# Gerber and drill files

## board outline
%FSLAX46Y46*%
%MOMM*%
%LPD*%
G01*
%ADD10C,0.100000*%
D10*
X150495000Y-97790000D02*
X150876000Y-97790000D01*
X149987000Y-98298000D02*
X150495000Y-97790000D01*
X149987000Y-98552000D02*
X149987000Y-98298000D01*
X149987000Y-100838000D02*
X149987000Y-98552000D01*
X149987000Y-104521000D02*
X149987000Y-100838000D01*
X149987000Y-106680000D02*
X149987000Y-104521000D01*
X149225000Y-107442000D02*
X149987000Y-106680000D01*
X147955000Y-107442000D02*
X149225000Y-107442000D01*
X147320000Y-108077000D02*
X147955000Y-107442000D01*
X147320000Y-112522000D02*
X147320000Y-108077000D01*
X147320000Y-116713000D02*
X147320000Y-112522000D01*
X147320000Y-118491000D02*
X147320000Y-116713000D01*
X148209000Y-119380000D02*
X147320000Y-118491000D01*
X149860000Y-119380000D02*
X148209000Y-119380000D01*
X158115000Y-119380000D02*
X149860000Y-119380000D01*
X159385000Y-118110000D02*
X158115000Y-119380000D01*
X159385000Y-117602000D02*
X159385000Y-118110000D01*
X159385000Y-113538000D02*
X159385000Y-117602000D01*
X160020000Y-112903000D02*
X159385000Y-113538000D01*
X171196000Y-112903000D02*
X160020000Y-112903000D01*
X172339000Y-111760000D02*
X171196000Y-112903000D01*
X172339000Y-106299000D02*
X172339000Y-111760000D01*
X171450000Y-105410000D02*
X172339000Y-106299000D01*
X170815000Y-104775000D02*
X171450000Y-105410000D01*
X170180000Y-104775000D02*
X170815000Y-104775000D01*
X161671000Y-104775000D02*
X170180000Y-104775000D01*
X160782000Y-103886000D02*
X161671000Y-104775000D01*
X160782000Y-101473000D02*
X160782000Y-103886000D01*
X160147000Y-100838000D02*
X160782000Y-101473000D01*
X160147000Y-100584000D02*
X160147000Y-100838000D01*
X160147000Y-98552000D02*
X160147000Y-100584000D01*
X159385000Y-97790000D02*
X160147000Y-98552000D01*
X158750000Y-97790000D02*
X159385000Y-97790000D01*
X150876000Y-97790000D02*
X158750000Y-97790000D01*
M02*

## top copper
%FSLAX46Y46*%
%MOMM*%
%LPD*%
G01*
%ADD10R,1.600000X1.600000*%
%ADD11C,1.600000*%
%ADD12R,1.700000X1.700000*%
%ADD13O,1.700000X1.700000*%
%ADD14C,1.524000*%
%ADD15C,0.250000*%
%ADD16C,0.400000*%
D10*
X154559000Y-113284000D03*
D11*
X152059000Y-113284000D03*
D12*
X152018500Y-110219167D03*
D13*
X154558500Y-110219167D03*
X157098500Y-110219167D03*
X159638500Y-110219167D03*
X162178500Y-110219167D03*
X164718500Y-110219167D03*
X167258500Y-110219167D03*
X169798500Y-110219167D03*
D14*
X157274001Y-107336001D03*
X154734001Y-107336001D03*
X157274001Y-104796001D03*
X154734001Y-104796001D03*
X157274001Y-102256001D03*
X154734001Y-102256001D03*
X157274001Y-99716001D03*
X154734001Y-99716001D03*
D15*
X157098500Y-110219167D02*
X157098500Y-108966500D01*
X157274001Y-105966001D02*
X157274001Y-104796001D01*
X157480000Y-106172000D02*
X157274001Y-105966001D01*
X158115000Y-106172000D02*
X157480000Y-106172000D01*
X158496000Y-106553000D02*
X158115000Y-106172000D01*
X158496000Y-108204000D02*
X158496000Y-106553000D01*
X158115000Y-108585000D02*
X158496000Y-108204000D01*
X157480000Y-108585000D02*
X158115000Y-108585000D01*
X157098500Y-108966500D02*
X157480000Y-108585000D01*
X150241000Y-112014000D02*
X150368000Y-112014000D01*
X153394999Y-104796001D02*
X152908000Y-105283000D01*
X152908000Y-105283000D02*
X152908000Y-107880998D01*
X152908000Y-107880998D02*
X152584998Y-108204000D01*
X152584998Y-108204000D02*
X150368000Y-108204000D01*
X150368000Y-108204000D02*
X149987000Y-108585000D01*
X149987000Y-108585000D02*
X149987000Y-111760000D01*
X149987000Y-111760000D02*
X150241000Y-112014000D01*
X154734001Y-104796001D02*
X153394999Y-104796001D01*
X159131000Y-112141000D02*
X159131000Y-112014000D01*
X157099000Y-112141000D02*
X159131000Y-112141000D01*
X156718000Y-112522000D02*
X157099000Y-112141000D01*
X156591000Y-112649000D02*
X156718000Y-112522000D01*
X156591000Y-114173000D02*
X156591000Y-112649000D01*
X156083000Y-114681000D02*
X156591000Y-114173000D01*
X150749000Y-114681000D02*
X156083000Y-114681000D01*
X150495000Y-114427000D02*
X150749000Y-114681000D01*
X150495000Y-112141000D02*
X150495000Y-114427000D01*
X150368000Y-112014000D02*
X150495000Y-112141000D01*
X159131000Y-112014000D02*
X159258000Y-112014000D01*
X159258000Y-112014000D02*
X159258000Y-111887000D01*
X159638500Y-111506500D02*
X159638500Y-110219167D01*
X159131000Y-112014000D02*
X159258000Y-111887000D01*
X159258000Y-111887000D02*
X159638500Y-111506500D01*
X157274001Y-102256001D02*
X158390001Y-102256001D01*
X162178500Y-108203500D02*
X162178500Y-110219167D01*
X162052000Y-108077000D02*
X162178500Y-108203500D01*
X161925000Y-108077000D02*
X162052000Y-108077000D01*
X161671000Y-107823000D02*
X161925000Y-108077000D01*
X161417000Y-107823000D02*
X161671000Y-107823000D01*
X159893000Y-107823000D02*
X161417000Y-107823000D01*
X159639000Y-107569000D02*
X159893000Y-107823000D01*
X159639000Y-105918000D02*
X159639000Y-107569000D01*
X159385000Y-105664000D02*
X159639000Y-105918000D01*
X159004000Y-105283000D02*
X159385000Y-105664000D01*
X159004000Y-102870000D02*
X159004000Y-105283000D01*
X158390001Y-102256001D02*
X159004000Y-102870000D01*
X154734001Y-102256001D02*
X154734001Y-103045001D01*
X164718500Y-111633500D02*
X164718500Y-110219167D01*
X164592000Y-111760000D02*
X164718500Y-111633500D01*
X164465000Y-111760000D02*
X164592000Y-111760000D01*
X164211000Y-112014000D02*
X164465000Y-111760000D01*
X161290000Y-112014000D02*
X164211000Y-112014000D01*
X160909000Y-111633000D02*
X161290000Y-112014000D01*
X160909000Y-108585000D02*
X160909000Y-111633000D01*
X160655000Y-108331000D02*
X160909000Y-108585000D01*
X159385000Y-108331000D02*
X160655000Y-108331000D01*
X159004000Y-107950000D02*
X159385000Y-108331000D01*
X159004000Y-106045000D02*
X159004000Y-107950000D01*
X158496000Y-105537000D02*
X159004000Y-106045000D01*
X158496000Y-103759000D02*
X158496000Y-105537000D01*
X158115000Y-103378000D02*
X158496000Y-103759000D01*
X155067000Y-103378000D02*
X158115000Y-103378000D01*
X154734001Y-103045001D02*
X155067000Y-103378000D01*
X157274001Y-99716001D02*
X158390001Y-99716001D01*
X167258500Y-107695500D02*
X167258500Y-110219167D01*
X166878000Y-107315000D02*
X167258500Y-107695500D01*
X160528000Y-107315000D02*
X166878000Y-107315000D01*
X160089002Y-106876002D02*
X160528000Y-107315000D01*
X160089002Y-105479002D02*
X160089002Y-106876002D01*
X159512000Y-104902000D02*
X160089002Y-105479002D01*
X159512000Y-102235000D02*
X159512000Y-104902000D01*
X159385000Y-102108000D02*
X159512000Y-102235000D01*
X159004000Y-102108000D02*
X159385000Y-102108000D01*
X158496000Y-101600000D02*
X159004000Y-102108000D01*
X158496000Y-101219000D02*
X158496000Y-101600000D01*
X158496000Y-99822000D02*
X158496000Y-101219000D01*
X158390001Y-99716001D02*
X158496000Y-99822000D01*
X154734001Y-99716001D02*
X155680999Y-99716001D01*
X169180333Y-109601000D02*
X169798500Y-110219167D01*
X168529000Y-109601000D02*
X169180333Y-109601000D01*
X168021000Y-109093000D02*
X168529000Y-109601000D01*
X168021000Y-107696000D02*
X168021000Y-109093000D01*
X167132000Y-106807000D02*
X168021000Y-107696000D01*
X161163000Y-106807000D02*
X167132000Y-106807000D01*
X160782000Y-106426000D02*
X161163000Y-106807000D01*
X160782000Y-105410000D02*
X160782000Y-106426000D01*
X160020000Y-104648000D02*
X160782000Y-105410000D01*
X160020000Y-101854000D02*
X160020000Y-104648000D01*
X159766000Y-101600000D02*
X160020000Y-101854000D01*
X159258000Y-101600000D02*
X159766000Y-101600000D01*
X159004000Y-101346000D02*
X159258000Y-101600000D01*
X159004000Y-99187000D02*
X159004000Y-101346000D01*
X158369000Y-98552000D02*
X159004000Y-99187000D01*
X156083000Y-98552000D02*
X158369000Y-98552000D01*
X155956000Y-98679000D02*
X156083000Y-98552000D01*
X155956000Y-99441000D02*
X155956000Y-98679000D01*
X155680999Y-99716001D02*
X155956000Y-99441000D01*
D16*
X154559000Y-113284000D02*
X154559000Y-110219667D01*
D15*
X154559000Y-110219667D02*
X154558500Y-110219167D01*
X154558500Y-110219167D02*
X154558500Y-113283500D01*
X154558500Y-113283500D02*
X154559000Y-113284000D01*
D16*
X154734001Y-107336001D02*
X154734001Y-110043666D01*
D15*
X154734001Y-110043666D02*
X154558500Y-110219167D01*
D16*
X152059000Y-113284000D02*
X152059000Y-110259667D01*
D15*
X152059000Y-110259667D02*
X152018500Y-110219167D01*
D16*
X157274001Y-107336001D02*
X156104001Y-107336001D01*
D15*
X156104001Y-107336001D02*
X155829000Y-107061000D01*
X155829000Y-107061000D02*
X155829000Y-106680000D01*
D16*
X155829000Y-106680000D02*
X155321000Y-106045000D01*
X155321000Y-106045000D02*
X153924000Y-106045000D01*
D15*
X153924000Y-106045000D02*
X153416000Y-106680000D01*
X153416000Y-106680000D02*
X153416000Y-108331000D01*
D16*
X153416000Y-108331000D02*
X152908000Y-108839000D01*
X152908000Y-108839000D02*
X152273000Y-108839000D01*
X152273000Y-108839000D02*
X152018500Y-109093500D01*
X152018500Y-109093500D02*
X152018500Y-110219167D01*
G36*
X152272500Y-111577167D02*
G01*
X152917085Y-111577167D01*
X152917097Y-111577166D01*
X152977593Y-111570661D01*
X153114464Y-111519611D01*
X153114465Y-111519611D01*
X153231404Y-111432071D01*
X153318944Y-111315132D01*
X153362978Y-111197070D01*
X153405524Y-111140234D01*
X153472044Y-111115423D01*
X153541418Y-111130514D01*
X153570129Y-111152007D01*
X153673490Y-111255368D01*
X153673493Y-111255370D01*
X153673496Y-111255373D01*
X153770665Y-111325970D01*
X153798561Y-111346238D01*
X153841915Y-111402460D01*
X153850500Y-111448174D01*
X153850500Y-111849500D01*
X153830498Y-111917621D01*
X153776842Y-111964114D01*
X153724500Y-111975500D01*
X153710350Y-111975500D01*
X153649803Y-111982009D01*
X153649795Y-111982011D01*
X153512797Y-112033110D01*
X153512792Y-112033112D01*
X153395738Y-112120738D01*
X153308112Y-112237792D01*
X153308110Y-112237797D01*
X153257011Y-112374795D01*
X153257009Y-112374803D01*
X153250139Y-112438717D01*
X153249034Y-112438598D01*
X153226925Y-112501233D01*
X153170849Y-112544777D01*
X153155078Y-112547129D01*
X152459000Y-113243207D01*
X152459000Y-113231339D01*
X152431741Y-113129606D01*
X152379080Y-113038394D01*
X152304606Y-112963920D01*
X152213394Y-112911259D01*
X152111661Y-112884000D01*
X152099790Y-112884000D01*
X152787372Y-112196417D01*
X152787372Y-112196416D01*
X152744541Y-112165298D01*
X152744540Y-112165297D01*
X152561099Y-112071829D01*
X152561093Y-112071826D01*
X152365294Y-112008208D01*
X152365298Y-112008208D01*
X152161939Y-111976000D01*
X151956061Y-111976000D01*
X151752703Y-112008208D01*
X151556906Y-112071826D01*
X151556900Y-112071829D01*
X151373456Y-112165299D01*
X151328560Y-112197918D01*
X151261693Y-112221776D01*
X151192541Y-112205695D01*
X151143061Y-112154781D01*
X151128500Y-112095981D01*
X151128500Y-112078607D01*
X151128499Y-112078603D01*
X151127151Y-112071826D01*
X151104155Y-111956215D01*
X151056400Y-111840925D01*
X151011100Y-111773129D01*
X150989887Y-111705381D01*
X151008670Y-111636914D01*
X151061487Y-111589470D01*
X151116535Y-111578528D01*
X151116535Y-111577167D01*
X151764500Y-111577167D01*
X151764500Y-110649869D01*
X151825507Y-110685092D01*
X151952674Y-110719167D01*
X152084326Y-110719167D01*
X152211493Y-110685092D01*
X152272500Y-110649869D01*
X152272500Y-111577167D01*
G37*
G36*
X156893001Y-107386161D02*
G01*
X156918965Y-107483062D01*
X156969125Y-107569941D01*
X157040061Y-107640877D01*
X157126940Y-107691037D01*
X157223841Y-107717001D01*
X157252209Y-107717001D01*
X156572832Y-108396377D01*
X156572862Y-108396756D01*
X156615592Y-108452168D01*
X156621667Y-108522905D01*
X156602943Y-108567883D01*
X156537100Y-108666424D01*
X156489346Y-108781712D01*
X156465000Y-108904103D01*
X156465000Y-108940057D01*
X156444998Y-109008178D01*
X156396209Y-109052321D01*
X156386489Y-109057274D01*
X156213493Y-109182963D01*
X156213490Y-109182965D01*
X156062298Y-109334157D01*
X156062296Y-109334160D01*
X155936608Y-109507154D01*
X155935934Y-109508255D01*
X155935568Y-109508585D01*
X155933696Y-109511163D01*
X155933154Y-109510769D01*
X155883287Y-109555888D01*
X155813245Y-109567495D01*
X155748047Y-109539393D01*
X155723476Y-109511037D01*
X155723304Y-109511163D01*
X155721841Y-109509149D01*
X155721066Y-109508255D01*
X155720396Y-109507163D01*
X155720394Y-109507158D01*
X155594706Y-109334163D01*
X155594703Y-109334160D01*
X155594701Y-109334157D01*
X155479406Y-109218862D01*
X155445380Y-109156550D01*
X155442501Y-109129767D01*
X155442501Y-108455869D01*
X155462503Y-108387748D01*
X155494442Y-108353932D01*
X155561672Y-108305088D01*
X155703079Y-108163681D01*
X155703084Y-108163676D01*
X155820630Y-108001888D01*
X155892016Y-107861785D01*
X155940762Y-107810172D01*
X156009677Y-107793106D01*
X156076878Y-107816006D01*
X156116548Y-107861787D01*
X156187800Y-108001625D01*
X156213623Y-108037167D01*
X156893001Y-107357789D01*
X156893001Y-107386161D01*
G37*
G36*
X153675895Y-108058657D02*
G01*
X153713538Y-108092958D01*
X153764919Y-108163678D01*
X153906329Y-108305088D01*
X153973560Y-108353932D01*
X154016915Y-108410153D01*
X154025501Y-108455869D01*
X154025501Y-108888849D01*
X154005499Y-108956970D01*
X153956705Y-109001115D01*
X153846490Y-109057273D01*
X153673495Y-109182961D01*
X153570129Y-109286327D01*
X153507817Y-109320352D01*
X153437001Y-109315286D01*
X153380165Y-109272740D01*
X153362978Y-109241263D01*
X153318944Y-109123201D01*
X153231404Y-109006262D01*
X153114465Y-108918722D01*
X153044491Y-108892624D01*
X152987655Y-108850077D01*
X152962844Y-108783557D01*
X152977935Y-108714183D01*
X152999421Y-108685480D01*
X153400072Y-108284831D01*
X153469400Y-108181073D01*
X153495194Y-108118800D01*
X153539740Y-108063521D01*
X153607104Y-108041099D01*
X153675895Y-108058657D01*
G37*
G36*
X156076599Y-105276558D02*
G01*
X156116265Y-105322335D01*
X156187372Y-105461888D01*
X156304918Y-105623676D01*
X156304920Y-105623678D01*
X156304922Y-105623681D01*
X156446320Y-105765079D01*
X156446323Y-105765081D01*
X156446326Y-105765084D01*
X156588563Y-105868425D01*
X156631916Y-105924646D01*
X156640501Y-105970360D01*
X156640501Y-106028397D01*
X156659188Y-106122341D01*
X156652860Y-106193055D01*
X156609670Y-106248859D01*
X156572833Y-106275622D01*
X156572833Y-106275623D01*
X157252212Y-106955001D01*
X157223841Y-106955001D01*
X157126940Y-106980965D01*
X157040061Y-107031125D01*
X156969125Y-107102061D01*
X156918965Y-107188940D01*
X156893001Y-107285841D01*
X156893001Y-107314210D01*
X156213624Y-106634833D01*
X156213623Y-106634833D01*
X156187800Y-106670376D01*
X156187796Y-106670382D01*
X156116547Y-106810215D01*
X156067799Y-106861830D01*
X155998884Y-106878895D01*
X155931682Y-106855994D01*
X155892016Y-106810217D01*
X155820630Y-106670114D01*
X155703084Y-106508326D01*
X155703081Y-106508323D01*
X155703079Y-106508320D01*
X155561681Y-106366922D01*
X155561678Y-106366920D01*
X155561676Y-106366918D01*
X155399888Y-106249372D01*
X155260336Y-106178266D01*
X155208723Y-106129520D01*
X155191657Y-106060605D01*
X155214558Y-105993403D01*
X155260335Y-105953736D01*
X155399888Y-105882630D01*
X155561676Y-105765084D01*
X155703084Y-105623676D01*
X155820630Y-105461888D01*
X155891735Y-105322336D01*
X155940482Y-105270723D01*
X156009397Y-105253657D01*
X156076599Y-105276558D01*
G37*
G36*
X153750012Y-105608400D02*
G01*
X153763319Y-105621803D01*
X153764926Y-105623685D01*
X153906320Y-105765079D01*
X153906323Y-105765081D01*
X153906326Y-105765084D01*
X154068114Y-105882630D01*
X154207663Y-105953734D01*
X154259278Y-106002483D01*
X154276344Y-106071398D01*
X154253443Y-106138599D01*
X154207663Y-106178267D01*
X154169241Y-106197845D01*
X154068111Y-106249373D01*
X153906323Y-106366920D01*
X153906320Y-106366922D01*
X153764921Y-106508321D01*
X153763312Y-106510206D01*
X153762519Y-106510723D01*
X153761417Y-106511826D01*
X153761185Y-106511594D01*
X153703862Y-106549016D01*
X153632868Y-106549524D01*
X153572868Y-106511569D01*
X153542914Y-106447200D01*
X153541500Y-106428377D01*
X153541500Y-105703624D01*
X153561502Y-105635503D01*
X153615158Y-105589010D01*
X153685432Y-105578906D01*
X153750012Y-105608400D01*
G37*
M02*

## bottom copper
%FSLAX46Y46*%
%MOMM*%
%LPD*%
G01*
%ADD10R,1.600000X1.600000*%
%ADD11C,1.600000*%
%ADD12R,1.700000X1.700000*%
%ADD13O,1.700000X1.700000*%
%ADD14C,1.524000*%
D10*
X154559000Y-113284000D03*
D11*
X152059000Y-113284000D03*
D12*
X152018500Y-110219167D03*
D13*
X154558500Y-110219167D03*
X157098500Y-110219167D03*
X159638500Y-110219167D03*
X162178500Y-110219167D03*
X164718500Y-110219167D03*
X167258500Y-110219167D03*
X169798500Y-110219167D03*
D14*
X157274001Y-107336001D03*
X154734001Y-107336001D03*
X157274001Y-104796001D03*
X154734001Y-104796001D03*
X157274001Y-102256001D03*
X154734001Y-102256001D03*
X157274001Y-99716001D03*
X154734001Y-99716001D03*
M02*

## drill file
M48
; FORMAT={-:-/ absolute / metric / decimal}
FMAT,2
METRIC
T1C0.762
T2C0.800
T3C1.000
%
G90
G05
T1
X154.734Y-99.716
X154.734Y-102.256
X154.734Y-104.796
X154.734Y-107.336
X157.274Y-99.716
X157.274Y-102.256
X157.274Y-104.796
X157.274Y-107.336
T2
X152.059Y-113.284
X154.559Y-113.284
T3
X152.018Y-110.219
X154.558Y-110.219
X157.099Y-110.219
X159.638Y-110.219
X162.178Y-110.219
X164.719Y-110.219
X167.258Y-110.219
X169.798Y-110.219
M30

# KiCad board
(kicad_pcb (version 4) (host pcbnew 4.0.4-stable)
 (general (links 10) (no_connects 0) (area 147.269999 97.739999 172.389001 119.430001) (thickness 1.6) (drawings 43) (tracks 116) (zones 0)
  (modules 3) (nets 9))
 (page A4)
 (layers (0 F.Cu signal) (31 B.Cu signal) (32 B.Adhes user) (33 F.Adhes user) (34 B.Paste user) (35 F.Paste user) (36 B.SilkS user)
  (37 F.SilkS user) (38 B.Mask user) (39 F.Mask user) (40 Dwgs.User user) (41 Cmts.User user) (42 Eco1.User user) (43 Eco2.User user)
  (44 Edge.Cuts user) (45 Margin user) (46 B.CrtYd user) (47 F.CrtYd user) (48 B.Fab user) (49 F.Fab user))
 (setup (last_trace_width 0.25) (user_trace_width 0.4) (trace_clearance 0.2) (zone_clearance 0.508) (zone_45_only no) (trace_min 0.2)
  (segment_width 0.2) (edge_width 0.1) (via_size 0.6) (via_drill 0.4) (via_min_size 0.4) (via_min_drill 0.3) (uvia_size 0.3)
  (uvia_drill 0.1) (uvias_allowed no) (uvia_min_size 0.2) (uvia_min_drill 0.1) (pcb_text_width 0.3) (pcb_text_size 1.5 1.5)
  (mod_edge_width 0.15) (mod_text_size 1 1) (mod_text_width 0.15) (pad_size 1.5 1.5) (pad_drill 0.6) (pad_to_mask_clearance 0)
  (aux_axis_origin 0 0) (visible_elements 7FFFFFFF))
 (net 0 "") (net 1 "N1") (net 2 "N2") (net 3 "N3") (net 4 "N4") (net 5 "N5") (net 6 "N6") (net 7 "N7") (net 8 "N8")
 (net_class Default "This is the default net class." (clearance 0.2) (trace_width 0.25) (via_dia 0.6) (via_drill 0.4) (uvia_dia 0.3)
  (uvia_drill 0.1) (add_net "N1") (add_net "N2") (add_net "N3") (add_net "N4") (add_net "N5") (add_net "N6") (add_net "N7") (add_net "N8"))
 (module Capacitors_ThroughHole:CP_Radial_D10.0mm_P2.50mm (layer F.Cu) (at 154.559 113.284 180)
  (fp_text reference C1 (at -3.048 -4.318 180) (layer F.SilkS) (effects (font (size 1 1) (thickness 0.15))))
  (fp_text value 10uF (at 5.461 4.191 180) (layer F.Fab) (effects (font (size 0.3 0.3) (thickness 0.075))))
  (pad 1 thru_hole rect (at 0 0 180) (size 1.6 1.6) (drill 0.8) (layers *.Cu *.Mask) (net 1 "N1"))
  (pad 2 thru_hole circle (at 2.5 0 180) (size 1.6 1.6) (drill 0.8) (layers *.Cu *.Mask) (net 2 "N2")))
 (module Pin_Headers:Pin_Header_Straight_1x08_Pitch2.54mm (layer F.Cu) (at 152.0185 110.219167 90)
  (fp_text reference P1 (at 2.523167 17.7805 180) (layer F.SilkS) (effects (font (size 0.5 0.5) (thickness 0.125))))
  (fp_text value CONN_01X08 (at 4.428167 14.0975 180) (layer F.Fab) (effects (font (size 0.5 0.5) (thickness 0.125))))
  (pad 1 thru_hole rect (at 0 0 90) (size 1.7 1.7) (drill 1) (layers *.Cu *.Mask) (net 2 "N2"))
  (pad 2 thru_hole oval (at 0 2.54 90) (size 1.7 1.7) (drill 1) (layers *.Cu *.Mask) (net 1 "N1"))
  (pad 3 thru_hole oval (at 0 5.08 90) (size 1.7 1.7) (drill 1) (layers *.Cu *.Mask) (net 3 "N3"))
  (pad 4 thru_hole oval (at 0 7.62 90) (size 1.7 1.7) (drill 1) (layers *.Cu *.Mask) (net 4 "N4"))
  (pad 5 thru_hole oval (at 0 10.16 90) (size 1.7 1.7) (drill 1) (layers *.Cu *.Mask) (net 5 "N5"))
  (pad 6 thru_hole oval (at 0 12.7 90) (size 1.7 1.7) (drill 1) (layers *.Cu *.Mask) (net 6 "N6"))
  (pad 7 thru_hole oval (at 0 15.24 90) (size 1.7 1.7) (drill 1) (layers *.Cu *.Mask) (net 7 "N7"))
  (pad 8 thru_hole oval (at 0 17.78 90) (size 1.7 1.7) (drill 1) (layers *.Cu *.Mask) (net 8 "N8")))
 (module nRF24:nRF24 (layer F.Cu) (at 154.734001 103.780001)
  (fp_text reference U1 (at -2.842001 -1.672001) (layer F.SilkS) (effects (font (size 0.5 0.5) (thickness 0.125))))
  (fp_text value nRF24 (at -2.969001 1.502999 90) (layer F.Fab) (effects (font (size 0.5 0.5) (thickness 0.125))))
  (pad 1 thru_hole circle (at 2.54 3.556) (size 1.524 1.524) (drill 0.762) (layers *.Cu *.Mask) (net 2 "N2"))
  (pad 2 thru_hole circle (at 0 3.556) (size 1.524 1.524) (drill 0.762) (layers *.Cu *.Mask) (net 1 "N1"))
  (pad 3 thru_hole circle (at 2.54 1.016) (size 1.524 1.524) (drill 0.762) (layers *.Cu *.Mask) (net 3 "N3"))
  (pad 4 thru_hole circle (at 0 1.016) (size 1.524 1.524) (drill 0.762) (layers *.Cu *.Mask) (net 4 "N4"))
  (pad 5 thru_hole circle (at 2.54 -1.524) (size 1.524 1.524) (drill 0.762) (layers *.Cu *.Mask) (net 5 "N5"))
  (pad 6 thru_hole circle (at 0 -1.524) (size 1.524 1.524) (drill 0.762) (layers *.Cu *.Mask) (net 6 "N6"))
  (pad 7 thru_hole circle (at 2.54 -4.064) (size 1.524 1.524) (drill 0.762) (layers *.Cu *.Mask) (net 7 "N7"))
  (pad 8 thru_hole circle (at 0 -4.064) (size 1.524 1.524) (drill 0.762) (layers *.Cu *.Mask) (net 8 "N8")))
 (gr_line (start 150.495 97.79) (end 150.876 97.79) (angle 90) (layer Edge.Cuts) (width 0.1))
 (gr_line (start 149.987 98.298) (end 150.495 97.79) (angle 90) (layer Edge.Cuts) (width 0.1))
 (gr_line (start 149.987 98.552) (end 149.987 98.298) (angle 90) (layer Edge.Cuts) (width 0.1))
 (gr_line (start 149.987 100.838) (end 149.987 98.552) (angle 90) (layer Edge.Cuts) (width 0.1))
 (gr_line (start 149.987 104.521) (end 149.987 100.838) (angle 90) (layer Edge.Cuts) (width 0.1))
 (gr_line (start 149.987 106.68) (end 149.987 104.521) (angle 90) (layer Edge.Cuts) (width 0.1))
 (gr_line (start 149.225 107.442) (end 149.987 106.68) (angle 90) (layer Edge.Cuts) (width 0.1))
 (gr_line (start 147.955 107.442) (end 149.225 107.442) (angle 90) (layer Edge.Cuts) (width 0.1))
 (gr_line (start 147.32 108.077) (end 147.955 107.442) (angle 90) (layer Edge.Cuts) (width 0.1))
 (gr_line (start 147.32 112.522) (end 147.32 108.077) (angle 90) (layer Edge.Cuts) (width 0.1))
 (gr_line (start 147.32 116.713) (end 147.32 112.522) (angle 90) (layer Edge.Cuts) (width 0.1))
 (gr_line (start 147.32 118.491) (end 147.32 116.713) (angle 90) (layer Edge.Cuts) (width 0.1))
 (gr_line (start 148.209 119.38) (end 147.32 118.491) (angle 90) (layer Edge.Cuts) (width 0.1))
 (gr_line (start 149.86 119.38) (end 148.209 119.38) (angle 90) (layer Edge.Cuts) (width 0.1))
 (gr_line (start 158.115 119.38) (end 149.86 119.38) (angle 90) (layer Edge.Cuts) (width 0.1))
 (gr_line (start 159.385 118.11) (end 158.115 119.38) (angle 90) (layer Edge.Cuts) (width 0.1))
 (gr_line (start 159.385 117.602) (end 159.385 118.11) (angle 90) (layer Edge.Cuts) (width 0.1))
 (gr_line (start 159.385 113.538) (end 159.385 117.602) (angle 90) (layer Edge.Cuts) (width 0.1))
 (gr_line (start 160.02 112.903) (end 159.385 113.538) (angle 90) (layer Edge.Cuts) (width 0.1))
 (gr_line (start 171.196 112.903) (end 160.02 112.903) (angle 90) (layer Edge.Cuts) (width 0.1))
 (gr_line (start 172.339 111.76) (end 171.196 112.903) (angle 90) (layer Edge.Cuts) (width 0.1))
 (gr_line (start 172.339 106.299) (end 172.339 111.76) (angle 90) (layer Edge.Cuts) (width 0.1))
 (gr_line (start 171.45 105.41) (end 172.339 106.299) (angle 90) (layer Edge.Cuts) (width 0.1))
 (gr_line (start 170.815 104.775) (end 171.45 105.41) (angle 90) (layer Edge.Cuts) (width 0.1))
 (gr_line (start 170.18 104.775) (end 170.815 104.775) (angle 90) (layer Edge.Cuts) (width 0.1))
 (gr_line (start 161.671 104.775) (end 170.18 104.775) (angle 90) (layer Edge.Cuts) (width 0.1))
 (gr_line (start 160.782 103.886) (end 161.671 104.775) (angle 90) (layer Edge.Cuts) (width 0.1))
 (gr_line (start 160.782 101.473) (end 160.782 103.886) (angle 90) (layer Edge.Cuts) (width 0.1))
 (gr_line (start 160.147 100.838) (end 160.782 101.473) (angle 90) (layer Edge.Cuts) (width 0.1))
 (gr_line (start 160.147 100.584) (end 160.147 100.838) (angle 90) (layer Edge.Cuts) (width 0.1))
 (gr_line (start 160.147 98.552) (end 160.147 100.584) (angle 90) (layer Edge.Cuts) (width 0.1))
 (gr_line (start 159.385 97.79) (end 160.147 98.552) (angle 90) (layer Edge.Cuts) (width 0.1))
 (gr_line (start 158.75 97.79) (end 159.385 97.79) (angle 90) (layer Edge.Cuts) (width 0.1))
 (gr_line (start 150.876 97.79) (end 158.75 97.79) (angle 90) (layer Edge.Cuts) (width 0.1))
 (segment (start 157.0985 110.219167) (end 157.0985 108.9665) (width 0.25) (layer F.Cu) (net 3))
 (segment (start 157.274001 105.966001) (end 157.274001 104.796001) (width 0.25) (layer F.Cu) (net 3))
 (segment (start 157.48 106.172) (end 157.274001 105.966001) (width 0.25) (layer F.Cu) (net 3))
 (segment (start 158.115 106.172) (end 157.48 106.172) (width 0.25) (layer F.Cu) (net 3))
 (segment (start 158.496 106.553) (end 158.115 106.172) (width 0.25) (layer F.Cu) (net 3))
 (segment (start 158.496 108.204) (end 158.496 106.553) (width 0.25) (layer F.Cu) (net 3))
 (segment (start 158.115 108.585) (end 158.496 108.204) (width 0.25) (layer F.Cu) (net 3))
 (segment (start 157.48 108.585) (end 158.115 108.585) (width 0.25) (layer F.Cu) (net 3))
 (segment (start 157.0985 108.9665) (end 157.48 108.585) (width 0.25) (layer F.Cu) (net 3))
 (segment (start 150.241 112.014) (end 150.368 112.014) (width 0.25) (layer F.Cu) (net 4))
 (segment (start 153.394999 104.796001) (end 152.908 105.283) (width 0.25) (layer F.Cu) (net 4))
 (segment (start 152.908 105.283) (end 152.908 107.880998) (width 0.25) (layer F.Cu) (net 4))
 (segment (start 152.908 107.880998) (end 152.584998 108.204) (width 0.25) (layer F.Cu) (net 4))
 (segment (start 152.584998 108.204) (end 150.368 108.204) (width 0.25) (layer F.Cu) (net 4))
 (segment (start 150.368 108.204) (end 149.987 108.585) (width 0.25) (layer F.Cu) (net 4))
 (segment (start 149.987 108.585) (end 149.987 111.76) (width 0.25) (layer F.Cu) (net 4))
 (segment (start 149.987 111.76) (end 150.241 112.014) (width 0.25) (layer F.Cu) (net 4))
 (segment (start 154.734001 104.796001) (end 153.394999 104.796001) (width 0.25) (layer F.Cu) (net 4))
 (segment (start 159.131 112.141) (end 159.131 112.014) (width 0.25) (layer F.Cu) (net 4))
 (segment (start 157.099 112.141) (end 159.131 112.141) (width 0.25) (layer F.Cu) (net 4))
 (segment (start 156.718 112.522) (end 157.099 112.141) (width 0.25) (layer F.Cu) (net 4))
 (segment (start 156.591 112.649) (end 156.718 112.522) (width 0.25) (layer F.Cu) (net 4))
 (segment (start 156.591 114.173) (end 156.591 112.649) (width 0.25) (layer F.Cu) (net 4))
 (segment (start 156.083 114.681) (end 156.591 114.173) (width 0.25) (layer F.Cu) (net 4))
 (segment (start 150.749 114.681) (end 156.083 114.681) (width 0.25) (layer F.Cu) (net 4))
 (segment (start 150.495 114.427) (end 150.749 114.681) (width 0.25) (layer F.Cu) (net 4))
 (segment (start 150.495 112.141) (end 150.495 114.427) (width 0.25) (layer F.Cu) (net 4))
 (segment (start 150.368 112.014) (end 150.495 112.141) (width 0.25) (layer F.Cu) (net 4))
 (segment (start 159.131 112.014) (end 159.258 112.014) (width 0.25) (layer F.Cu) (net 4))
 (segment (start 159.258 112.014) (end 159.258 111.887) (width 0.25) (layer F.Cu) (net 4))
 (segment (start 159.6385 111.5065) (end 159.6385 110.219167) (width 0.25) (layer F.Cu) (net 4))
 (segment (start 159.131 112.014) (end 159.258 111.887) (width 0.25) (layer F.Cu) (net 4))
 (segment (start 159.258 111.887) (end 159.6385 111.5065) (width 0.25) (layer F.Cu) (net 4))
 (segment (start 157.274001 102.256001) (end 158.390001 102.256001) (width 0.25) (layer F.Cu) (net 5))
 (segment (start 162.1785 108.2035) (end 162.1785 110.219167) (width 0.25) (layer F.Cu) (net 5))
 (segment (start 162.052 108.077) (end 162.1785 108.2035) (width 0.25) (layer F.Cu) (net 5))
 (segment (start 161.925 108.077) (end 162.052 108.077) (width 0.25) (layer F.Cu) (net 5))
 (segment (start 161.671 107.823) (end 161.925 108.077) (width 0.25) (layer F.Cu) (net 5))
 (segment (start 161.417 107.823) (end 161.671 107.823) (width 0.25) (layer F.Cu) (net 5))
 (segment (start 159.893 107.823) (end 161.417 107.823) (width 0.25) (layer F.Cu) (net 5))
 (segment (start 159.639 107.569) (end 159.893 107.823) (width 0.25) (layer F.Cu) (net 5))
 (segment (start 159.639 105.918) (end 159.639 107.569) (width 0.25) (layer F.Cu) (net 5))
 (segment (start 159.385 105.664) (end 159.639 105.918) (width 0.25) (layer F.Cu) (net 5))
 (segment (start 159.004 105.283) (end 159.385 105.664) (width 0.25) (layer F.Cu) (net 5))
 (segment (start 159.004 102.87) (end 159.004 105.283) (width 0.25) (layer F.Cu) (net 5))
 (segment (start 158.390001 102.256001) (end 159.004 102.87) (width 0.25) (layer F.Cu) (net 5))
 (segment (start 154.734001 102.256001) (end 154.734001 103.045001) (width 0.25) (layer F.Cu) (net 6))
 (segment (start 164.7185 111.6335) (end 164.7185 110.219167) (width 0.25) (layer F.Cu) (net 6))
 (segment (start 164.592 111.76) (end 164.7185 111.6335) (width 0.25) (layer F.Cu) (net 6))
 (segment (start 164.465 111.76) (end 164.592 111.76) (width 0.25) (layer F.Cu) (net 6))
 (segment (start 164.211 112.014) (end 164.465 111.76) (width 0.25) (layer F.Cu) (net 6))
 (segment (start 161.29 112.014) (end 164.211 112.014) (width 0.25) (layer F.Cu) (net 6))
 (segment (start 160.909 111.633) (end 161.29 112.014) (width 0.25) (layer F.Cu) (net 6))
 (segment (start 160.909 108.585) (end 160.909 111.633) (width 0.25) (layer F.Cu) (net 6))
 (segment (start 160.655 108.331) (end 160.909 108.585) (width 0.25) (layer F.Cu) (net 6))
 (segment (start 159.385 108.331) (end 160.655 108.331) (width 0.25) (layer F.Cu) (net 6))
 (segment (start 159.004 107.95) (end 159.385 108.331) (width 0.25) (layer F.Cu) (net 6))
 (segment (start 159.004 106.045) (end 159.004 107.95) (width 0.25) (layer F.Cu) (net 6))
 (segment (start 158.496 105.537) (end 159.004 106.045) (width 0.25) (layer F.Cu) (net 6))
 (segment (start 158.496 103.759) (end 158.496 105.537) (width 0.25) (layer F.Cu) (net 6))
 (segment (start 158.115 103.378) (end 158.496 103.759) (width 0.25) (layer F.Cu) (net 6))
 (segment (start 155.067 103.378) (end 158.115 103.378) (width 0.25) (layer F.Cu) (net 6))
 (segment (start 154.734001 103.045001) (end 155.067 103.378) (width 0.25) (layer F.Cu) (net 6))
 (segment (start 157.274001 99.716001) (end 158.390001 99.716001) (width 0.25) (layer F.Cu) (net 7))
 (segment (start 167.2585 107.6955) (end 167.2585 110.219167) (width 0.25) (layer F.Cu) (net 7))
 (segment (start 166.878 107.315) (end 167.2585 107.6955) (width 0.25) (layer F.Cu) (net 7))
 (segment (start 160.528 107.315) (end 166.878 107.315) (width 0.25) (layer F.Cu) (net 7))
 (segment (start 160.089002 106.876002) (end 160.528 107.315) (width 0.25) (layer F.Cu) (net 7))
 (segment (start 160.089002 105.479002) (end 160.089002 106.876002) (width 0.25) (layer F.Cu) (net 7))
 (segment (start 159.512 104.902) (end 160.089002 105.479002) (width 0.25) (layer F.Cu) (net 7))
 (segment (start 159.512 102.235) (end 159.512 104.902) (width 0.25) (layer F.Cu) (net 7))
 (segment (start 159.385 102.108) (end 159.512 102.235) (width 0.25) (layer F.Cu) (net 7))
 (segment (start 159.004 102.108) (end 159.385 102.108) (width 0.25) (layer F.Cu) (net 7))
 (segment (start 158.496 101.6) (end 159.004 102.108) (width 0.25) (layer F.Cu) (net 7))
 (segment (start 158.496 101.219) (end 158.496 101.6) (width 0.25) (layer F.Cu) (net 7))
 (segment (start 158.496 99.822) (end 158.496 101.219) (width 0.25) (layer F.Cu) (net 7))
 (segment (start 158.390001 99.716001) (end 158.496 99.822) (width 0.25) (layer F.Cu) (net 7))
 (segment (start 154.734001 99.716001) (end 155.680999 99.716001) (width 0.25) (layer F.Cu) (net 8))
 (segment (start 169.180333 109.601) (end 169.7985 110.219167) (width 0.25) (layer F.Cu) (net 8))
 (segment (start 168.529 109.601) (end 169.180333 109.601) (width 0.25) (layer F.Cu) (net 8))
 (segment (start 168.021 109.093) (end 168.529 109.601) (width 0.25) (layer F.Cu) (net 8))
 (segment (start 168.021 107.696) (end 168.021 109.093) (width 0.25) (layer F.Cu) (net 8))
 (segment (start 167.132 106.807) (end 168.021 107.696) (width 0.25) (layer F.Cu) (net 8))
 (segment (start 161.163 106.807) (end 167.132 106.807) (width 0.25) (layer F.Cu) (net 8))
 (segment (start 160.782 106.426) (end 161.163 106.807) (width 0.25) (layer F.Cu) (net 8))
 (segment (start 160.782 105.41) (end 160.782 106.426) (width 0.25) (layer F.Cu) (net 8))
 (segment (start 160.02 104.648) (end 160.782 105.41) (width 0.25) (layer F.Cu) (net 8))
 (segment (start 160.02 101.854) (end 160.02 104.648) (width 0.25) (layer F.Cu) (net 8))
 (segment (start 159.766 101.6) (end 160.02 101.854) (width 0.25) (layer F.Cu) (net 8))
 (segment (start 159.258 101.6) (end 159.766 101.6) (width 0.25) (layer F.Cu) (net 8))
 (segment (start 159.004 101.346) (end 159.258 101.6) (width 0.25) (layer F.Cu) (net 8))
 (segment (start 159.004 99.187) (end 159.004 101.346) (width 0.25) (layer F.Cu) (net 8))
 (segment (start 158.369 98.552) (end 159.004 99.187) (width 0.25) (layer F.Cu) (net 8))
 (segment (start 156.083 98.552) (end 158.369 98.552) (width 0.25) (layer F.Cu) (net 8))
 (segment (start 155.956 98.679) (end 156.083 98.552) (width 0.25) (layer F.Cu) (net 8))
 (segment (start 155.956 99.441) (end 155.956 98.679) (width 0.25) (layer F.Cu) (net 8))
 (segment (start 155.680999 99.716001) (end 155.956 99.441) (width 0.25) (layer F.Cu) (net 8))
 (segment (start 154.559 113.284) (end 154.559 110.219667) (width 0.4) (layer F.Cu) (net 1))
 (segment (start 154.559 110.219667) (end 154.5585 110.219167) (width 0.25) (layer F.Cu) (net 1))
 (segment (start 154.5585 110.219167) (end 154.5585 113.2835) (width 0.25) (layer F.Cu) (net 1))
 (segment (start 154.5585 113.2835) (end 154.559 113.284) (width 0.25) (layer F.Cu) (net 1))
 (segment (start 154.734001 107.336001) (end 154.734001 110.043666) (width 0.4) (layer F.Cu) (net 1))
 (segment (start 154.734001 110.043666) (end 154.5585 110.219167) (width 0.25) (layer F.Cu) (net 1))
 (segment (start 152.059 113.284) (end 152.059 110.259667) (width 0.4) (layer F.Cu) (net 2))
 (segment (start 152.059 110.259667) (end 152.0185 110.219167) (width 0.25) (layer F.Cu) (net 2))
 (segment (start 157.274001 107.336001) (end 156.104001 107.336001) (width 0.4) (layer F.Cu) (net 2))
 (segment (start 156.104001 107.336001) (end 155.829 107.061) (width 0.25) (layer F.Cu) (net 2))
 (segment (start 155.829 107.061) (end 155.829 106.68) (width 0.25) (layer F.Cu) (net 2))
 (segment (start 155.829 106.68) (end 155.321 106.045) (width 0.4) (layer F.Cu) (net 2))
 (segment (start 155.321 106.045) (end 153.924 106.045) (width 0.4) (layer F.Cu) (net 2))
 (segment (start 153.924 106.045) (end 153.416 106.68) (width 0.25) (layer F.Cu) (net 2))
 (segment (start 153.416 106.68) (end 153.416 108.331) (width 0.25) (layer F.Cu) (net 2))
 (segment (start 153.416 108.331) (end 152.908 108.839) (width 0.4) (layer F.Cu) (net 2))
 (segment (start 152.908 108.839) (end 152.273 108.839) (width 0.4) (layer F.Cu) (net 2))
 (segment (start 152.273 108.839) (end 152.0185 109.0935) (width 0.4) (layer F.Cu) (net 2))
 (segment (start 152.0185 109.0935) (end 152.0185 110.219167) (width 0.4) (layer F.Cu) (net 2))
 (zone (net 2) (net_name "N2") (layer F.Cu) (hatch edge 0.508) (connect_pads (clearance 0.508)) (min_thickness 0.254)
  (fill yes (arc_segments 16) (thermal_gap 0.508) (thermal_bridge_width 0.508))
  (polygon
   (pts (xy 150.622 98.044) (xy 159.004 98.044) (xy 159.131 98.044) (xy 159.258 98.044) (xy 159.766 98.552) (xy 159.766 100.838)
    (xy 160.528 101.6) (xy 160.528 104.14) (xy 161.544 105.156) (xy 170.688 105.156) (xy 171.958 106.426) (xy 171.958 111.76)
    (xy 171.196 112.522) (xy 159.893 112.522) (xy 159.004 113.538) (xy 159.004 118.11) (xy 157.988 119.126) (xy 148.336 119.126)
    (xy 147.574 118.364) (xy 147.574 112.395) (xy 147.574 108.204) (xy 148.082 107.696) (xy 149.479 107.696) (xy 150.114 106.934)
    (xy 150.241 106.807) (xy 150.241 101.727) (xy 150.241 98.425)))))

